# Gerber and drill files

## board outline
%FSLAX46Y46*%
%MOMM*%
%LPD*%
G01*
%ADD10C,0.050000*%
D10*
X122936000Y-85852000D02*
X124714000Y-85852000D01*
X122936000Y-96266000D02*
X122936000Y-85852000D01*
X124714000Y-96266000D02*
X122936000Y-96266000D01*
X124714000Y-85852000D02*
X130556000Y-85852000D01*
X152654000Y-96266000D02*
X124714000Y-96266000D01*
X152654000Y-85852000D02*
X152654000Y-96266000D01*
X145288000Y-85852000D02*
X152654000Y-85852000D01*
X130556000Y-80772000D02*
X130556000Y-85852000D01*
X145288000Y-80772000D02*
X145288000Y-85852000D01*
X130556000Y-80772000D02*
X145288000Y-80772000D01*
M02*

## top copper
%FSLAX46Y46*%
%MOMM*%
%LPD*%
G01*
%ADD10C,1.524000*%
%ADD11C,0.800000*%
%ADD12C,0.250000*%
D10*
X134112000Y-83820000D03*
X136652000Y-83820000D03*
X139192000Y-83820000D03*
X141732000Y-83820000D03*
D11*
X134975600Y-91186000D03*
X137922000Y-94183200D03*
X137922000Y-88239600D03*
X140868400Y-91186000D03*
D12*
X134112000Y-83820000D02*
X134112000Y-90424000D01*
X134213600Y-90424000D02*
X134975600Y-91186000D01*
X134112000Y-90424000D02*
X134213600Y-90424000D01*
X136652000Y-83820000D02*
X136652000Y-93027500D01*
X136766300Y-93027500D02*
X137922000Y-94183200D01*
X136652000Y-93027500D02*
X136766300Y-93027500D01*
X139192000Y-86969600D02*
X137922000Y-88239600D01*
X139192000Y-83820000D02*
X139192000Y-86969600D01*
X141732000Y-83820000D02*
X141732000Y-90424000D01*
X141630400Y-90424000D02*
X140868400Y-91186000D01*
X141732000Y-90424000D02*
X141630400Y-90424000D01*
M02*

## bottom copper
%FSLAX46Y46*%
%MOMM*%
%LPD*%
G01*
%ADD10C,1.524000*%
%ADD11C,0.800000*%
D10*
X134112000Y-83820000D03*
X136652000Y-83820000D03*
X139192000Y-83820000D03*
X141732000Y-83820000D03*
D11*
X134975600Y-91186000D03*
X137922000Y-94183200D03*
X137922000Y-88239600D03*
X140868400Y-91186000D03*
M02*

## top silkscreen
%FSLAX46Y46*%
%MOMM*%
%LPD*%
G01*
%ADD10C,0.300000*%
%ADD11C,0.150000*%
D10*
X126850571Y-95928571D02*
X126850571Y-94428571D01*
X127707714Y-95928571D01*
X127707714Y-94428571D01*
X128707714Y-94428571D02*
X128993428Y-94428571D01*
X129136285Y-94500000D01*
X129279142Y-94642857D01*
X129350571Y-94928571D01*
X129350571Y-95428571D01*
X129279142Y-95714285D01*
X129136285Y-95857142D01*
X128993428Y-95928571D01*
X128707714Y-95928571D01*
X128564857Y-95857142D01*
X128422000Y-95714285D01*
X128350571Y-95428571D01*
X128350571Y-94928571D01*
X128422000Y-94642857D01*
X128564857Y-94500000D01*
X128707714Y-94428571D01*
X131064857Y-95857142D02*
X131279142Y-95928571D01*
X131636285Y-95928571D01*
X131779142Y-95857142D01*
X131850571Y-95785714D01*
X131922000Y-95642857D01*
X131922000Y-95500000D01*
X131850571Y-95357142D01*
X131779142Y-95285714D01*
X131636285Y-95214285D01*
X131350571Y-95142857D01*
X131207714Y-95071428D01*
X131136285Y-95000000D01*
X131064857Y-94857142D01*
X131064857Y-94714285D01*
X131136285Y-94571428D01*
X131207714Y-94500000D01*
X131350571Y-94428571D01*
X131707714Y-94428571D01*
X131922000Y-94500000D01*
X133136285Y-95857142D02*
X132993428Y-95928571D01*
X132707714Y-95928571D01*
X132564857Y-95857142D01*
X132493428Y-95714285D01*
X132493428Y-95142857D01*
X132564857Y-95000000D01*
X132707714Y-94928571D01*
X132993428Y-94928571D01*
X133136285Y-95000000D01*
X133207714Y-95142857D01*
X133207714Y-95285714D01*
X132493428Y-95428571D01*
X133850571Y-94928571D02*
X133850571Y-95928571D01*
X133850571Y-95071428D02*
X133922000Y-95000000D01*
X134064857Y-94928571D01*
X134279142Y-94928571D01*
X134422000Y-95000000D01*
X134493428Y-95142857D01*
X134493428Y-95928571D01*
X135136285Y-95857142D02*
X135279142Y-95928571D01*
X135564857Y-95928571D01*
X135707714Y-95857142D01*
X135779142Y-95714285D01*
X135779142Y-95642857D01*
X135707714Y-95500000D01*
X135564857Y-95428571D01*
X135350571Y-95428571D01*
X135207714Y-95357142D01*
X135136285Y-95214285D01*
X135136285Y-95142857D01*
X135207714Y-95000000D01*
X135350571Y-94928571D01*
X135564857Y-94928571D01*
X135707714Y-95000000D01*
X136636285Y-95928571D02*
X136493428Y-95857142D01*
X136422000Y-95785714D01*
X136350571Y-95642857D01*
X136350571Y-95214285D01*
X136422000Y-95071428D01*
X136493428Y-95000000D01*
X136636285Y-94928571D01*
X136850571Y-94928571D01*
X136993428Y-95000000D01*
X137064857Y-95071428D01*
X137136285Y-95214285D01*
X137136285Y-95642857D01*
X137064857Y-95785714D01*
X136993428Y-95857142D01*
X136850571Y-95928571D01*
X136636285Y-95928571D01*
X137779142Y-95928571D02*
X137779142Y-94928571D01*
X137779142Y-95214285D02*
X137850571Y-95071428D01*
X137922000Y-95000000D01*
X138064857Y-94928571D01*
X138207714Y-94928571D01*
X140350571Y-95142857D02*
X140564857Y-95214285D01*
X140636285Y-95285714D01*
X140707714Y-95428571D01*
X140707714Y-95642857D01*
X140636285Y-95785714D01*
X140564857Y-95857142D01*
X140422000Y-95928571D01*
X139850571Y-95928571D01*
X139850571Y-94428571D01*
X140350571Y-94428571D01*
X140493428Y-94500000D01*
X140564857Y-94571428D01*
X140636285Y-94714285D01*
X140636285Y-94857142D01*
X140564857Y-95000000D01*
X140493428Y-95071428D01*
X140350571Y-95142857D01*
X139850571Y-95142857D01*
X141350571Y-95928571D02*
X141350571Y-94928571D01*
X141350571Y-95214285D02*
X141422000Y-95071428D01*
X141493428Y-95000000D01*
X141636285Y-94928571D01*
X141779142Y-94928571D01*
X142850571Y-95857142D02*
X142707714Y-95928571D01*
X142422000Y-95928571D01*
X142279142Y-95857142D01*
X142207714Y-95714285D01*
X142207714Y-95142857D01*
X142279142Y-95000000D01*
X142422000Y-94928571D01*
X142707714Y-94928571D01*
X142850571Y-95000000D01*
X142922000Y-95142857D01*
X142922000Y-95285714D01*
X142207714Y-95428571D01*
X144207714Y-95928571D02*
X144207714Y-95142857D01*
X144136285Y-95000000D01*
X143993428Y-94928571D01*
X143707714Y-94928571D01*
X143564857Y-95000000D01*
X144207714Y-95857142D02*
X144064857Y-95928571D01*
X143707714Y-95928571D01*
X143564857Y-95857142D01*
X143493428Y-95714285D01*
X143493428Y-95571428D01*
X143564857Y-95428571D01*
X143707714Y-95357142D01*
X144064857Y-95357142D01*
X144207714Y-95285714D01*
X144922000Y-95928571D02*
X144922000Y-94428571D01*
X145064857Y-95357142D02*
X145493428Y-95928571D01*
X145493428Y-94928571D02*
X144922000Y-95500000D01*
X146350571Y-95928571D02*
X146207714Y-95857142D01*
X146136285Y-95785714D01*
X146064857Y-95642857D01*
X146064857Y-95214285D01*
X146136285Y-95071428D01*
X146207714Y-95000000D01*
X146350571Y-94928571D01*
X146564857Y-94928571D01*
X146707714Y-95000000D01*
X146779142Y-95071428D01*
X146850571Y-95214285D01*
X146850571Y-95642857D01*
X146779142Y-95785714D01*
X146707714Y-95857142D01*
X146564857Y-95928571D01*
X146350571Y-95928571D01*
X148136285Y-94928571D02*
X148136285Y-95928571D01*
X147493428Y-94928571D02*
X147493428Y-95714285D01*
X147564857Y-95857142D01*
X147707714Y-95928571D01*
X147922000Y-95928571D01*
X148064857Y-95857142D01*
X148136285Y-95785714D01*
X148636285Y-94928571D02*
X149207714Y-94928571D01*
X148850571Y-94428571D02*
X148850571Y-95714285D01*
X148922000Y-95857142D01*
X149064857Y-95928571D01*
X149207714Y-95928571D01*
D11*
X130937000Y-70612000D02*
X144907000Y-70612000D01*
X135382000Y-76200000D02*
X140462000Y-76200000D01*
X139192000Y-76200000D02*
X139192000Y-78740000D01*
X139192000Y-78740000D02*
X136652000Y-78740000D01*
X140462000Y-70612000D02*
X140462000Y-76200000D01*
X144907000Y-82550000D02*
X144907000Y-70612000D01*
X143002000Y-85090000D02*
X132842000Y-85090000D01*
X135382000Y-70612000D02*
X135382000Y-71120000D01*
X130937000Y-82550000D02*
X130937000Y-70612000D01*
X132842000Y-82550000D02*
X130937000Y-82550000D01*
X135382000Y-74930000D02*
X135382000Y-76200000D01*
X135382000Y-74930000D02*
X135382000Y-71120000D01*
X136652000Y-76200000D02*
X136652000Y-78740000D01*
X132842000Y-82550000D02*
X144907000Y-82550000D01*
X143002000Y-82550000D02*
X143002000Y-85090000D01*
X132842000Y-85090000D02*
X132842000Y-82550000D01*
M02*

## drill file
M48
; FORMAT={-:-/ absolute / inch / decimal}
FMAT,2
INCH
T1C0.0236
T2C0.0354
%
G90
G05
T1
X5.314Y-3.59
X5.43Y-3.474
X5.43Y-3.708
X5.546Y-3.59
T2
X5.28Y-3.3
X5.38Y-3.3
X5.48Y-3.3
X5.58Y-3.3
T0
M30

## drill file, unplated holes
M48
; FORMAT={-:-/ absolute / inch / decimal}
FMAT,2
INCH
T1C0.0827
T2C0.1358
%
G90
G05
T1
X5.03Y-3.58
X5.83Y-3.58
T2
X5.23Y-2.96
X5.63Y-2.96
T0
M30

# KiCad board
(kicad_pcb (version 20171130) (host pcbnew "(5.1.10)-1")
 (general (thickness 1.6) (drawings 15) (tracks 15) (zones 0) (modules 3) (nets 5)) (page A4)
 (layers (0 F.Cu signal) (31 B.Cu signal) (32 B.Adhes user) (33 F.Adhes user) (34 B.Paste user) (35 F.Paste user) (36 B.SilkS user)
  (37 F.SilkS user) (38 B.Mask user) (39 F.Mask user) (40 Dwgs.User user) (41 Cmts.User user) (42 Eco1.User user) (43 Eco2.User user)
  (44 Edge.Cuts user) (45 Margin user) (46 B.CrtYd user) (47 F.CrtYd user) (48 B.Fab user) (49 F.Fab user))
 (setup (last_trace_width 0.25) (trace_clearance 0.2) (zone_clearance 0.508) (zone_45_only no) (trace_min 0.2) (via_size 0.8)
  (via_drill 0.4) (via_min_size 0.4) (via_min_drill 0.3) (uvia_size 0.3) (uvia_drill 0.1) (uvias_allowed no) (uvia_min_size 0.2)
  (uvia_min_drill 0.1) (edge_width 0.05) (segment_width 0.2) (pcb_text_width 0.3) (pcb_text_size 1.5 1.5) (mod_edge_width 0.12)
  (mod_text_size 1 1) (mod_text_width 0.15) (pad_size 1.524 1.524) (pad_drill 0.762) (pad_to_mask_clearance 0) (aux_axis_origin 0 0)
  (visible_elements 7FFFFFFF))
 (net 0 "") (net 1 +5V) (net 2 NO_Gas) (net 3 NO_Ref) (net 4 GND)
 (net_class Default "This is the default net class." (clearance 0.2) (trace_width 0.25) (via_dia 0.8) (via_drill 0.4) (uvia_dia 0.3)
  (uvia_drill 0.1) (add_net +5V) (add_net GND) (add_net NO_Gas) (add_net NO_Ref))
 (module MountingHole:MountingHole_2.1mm (layer F.Cu) (at 127.762 90.932)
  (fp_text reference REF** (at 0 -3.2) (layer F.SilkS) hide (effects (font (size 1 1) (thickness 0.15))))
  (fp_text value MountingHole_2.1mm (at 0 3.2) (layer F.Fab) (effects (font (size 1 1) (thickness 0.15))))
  (pad "" np_thru_hole circle (at 0 0) (size 2.1 2.1) (drill 2.1) (layers *.Cu *.Mask)))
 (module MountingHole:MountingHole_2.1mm (layer F.Cu) (at 148.082 90.932)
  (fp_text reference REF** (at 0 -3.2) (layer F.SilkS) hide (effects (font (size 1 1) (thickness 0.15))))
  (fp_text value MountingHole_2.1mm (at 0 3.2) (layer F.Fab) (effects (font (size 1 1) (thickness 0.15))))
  (pad "" np_thru_hole circle (at 0 0) (size 2.1 2.1) (drill 2.1) (layers *.Cu *.Mask)))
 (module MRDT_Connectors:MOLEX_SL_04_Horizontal (layer F.Cu) (at 134.112 83.82)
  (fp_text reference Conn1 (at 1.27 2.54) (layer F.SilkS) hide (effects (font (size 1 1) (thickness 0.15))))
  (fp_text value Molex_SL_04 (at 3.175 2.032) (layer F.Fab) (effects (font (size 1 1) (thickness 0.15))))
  (fp_line (start -3.175 -13.208) (end 10.795 -13.208) (layer F.SilkS) (width 0.15))
  (fp_line (start 1.27 -7.62) (end 6.35 -7.62) (layer F.SilkS) (width 0.15))
  (fp_line (start 5.08 -7.62) (end 5.08 -5.08) (layer F.SilkS) (width 0.15))
  (fp_line (start 5.08 -5.08) (end 2.54 -5.08) (layer F.SilkS) (width 0.15))
  (fp_line (start 6.35 -13.208) (end 6.35 -7.62) (layer F.SilkS) (width 0.15))
  (fp_line (start 10.795 -1.27) (end 10.795 -13.208) (layer F.SilkS) (width 0.15))
  (fp_line (start 8.89 1.27) (end -1.27 1.27) (layer F.SilkS) (width 0.15))
  (fp_line (start 1.27 -13.208) (end 1.27 -12.7) (layer F.SilkS) (width 0.15))
  (fp_line (start -3.175 -1.27) (end -3.175 -13.208) (layer F.SilkS) (width 0.15))
  (fp_line (start -1.27 -1.27) (end -3.175 -1.27) (layer F.SilkS) (width 0.15))
  (fp_line (start 1.27 -8.89) (end 1.27 -7.62) (layer F.SilkS) (width 0.15))
  (fp_line (start 1.27 -8.89) (end 1.27 -12.7) (layer F.SilkS) (width 0.15))
  (fp_line (start 2.54 -7.62) (end 2.54 -5.08) (layer F.SilkS) (width 0.15))
  (fp_line (start -1.27 -1.27) (end 10.795 -1.27) (layer F.SilkS) (width 0.15))
  (fp_line (start 8.89 -1.27) (end 8.89 1.27) (layer F.SilkS) (width 0.15))
  (fp_line (start -1.27 1.27) (end -1.27 -1.27) (layer F.SilkS) (width 0.15))
  (pad 1 thru_hole circle (at 0 0) (size 1.524 1.524) (drill 0.9) (layers *.Cu *.Mask) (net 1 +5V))
  (pad 2 thru_hole circle (at 2.54 0) (size 1.524 1.524) (drill 0.9) (layers *.Cu *.Mask) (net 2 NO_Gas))
  (pad 3 thru_hole circle (at 5.08 0) (size 1.524 1.524) (drill 0.9) (layers *.Cu *.Mask) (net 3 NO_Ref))
  (pad 4 thru_hole circle (at 7.62 0) (size 1.524 1.524) (drill 0.9) (layers *.Cu *.Mask) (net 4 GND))
  (pad "" np_thru_hole circle (at -1.27 -8.636) (size 3.45 3.45) (drill 3.45) (layers *.Cu *.Mask))
  (pad "" np_thru_hole circle (at 8.89 -8.636) (size 3.45 3.45) (drill 3.45) (layers *.Cu *.Mask)))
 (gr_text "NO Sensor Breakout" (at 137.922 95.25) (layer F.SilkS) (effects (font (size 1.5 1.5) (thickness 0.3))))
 (gr_line (start 122.936 85.852) (end 124.714 85.852) (layer Edge.Cuts) (width 0.05))
 (gr_line (start 122.936 96.266) (end 122.936 85.852) (layer Edge.Cuts) (width 0.05))
 (gr_line (start 124.714 96.266) (end 122.936 96.266) (layer Edge.Cuts) (width 0.05))
 (gr_line (start 124.714 85.852) (end 130.556 85.852) (layer Edge.Cuts) (width 0.05))
 (gr_line (start 152.654 96.266) (end 124.714 96.266) (layer Edge.Cuts) (width 0.05))
 (gr_line (start 152.654 85.852) (end 152.654 96.266) (layer Edge.Cuts) (width 0.05))
 (gr_line (start 145.288 85.852) (end 152.654 85.852) (layer Edge.Cuts) (width 0.05))
 (gr_line (start 130.556 80.772) (end 130.556 85.852) (layer Edge.Cuts) (width 0.05))
 (gr_line (start 145.288 80.772) (end 145.288 85.852) (layer Edge.Cuts) (width 0.05))
 (gr_line (start 130.556 80.772) (end 145.288 80.772) (layer Edge.Cuts) (width 0.05))
 (via (at 134.9756 91.186) (size 0.8) (drill 0.6) (layers F.Cu B.Cu) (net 1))
 (segment (start 134.112 83.82) (end 134.112 90.424) (width 0.25) (layer F.Cu) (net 1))
 (segment (start 134.2136 90.424) (end 134.9756 91.186) (width 0.25) (layer F.Cu) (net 1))
 (segment (start 134.112 90.424) (end 134.2136 90.424) (width 0.25) (layer F.Cu) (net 1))
 (via (at 137.922 94.1832) (size 0.8) (drill 0.6) (layers F.Cu B.Cu) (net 2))
 (segment (start 136.652 83.82) (end 136.652 93.0275) (width 0.25) (layer F.Cu) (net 2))
 (segment (start 136.7663 93.0275) (end 137.922 94.1832) (width 0.25) (layer F.Cu) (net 2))
 (segment (start 136.652 93.0275) (end 136.7663 93.0275) (width 0.25) (layer F.Cu) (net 2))
 (via (at 137.922 88.2396) (size 0.8) (drill 0.6) (layers F.Cu B.Cu) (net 3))
 (segment (start 139.192 86.9696) (end 137.922 88.2396) (width 0.25) (layer F.Cu) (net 3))
 (segment (start 139.192 83.82) (end 139.192 86.9696) (width 0.25) (layer F.Cu) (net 3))
 (via (at 140.8684 91.186) (size 0.8) (drill 0.6) (layers F.Cu B.Cu) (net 4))
 (segment (start 141.732 83.82) (end 141.732 90.424) (width 0.25) (layer F.Cu) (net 4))
 (segment (start 141.6304 90.424) (end 140.8684 91.186) (width 0.25) (layer F.Cu) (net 4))
 (segment (start 141.732 90.424) (end 141.6304 90.424) (width 0.25) (layer F.Cu) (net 4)))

